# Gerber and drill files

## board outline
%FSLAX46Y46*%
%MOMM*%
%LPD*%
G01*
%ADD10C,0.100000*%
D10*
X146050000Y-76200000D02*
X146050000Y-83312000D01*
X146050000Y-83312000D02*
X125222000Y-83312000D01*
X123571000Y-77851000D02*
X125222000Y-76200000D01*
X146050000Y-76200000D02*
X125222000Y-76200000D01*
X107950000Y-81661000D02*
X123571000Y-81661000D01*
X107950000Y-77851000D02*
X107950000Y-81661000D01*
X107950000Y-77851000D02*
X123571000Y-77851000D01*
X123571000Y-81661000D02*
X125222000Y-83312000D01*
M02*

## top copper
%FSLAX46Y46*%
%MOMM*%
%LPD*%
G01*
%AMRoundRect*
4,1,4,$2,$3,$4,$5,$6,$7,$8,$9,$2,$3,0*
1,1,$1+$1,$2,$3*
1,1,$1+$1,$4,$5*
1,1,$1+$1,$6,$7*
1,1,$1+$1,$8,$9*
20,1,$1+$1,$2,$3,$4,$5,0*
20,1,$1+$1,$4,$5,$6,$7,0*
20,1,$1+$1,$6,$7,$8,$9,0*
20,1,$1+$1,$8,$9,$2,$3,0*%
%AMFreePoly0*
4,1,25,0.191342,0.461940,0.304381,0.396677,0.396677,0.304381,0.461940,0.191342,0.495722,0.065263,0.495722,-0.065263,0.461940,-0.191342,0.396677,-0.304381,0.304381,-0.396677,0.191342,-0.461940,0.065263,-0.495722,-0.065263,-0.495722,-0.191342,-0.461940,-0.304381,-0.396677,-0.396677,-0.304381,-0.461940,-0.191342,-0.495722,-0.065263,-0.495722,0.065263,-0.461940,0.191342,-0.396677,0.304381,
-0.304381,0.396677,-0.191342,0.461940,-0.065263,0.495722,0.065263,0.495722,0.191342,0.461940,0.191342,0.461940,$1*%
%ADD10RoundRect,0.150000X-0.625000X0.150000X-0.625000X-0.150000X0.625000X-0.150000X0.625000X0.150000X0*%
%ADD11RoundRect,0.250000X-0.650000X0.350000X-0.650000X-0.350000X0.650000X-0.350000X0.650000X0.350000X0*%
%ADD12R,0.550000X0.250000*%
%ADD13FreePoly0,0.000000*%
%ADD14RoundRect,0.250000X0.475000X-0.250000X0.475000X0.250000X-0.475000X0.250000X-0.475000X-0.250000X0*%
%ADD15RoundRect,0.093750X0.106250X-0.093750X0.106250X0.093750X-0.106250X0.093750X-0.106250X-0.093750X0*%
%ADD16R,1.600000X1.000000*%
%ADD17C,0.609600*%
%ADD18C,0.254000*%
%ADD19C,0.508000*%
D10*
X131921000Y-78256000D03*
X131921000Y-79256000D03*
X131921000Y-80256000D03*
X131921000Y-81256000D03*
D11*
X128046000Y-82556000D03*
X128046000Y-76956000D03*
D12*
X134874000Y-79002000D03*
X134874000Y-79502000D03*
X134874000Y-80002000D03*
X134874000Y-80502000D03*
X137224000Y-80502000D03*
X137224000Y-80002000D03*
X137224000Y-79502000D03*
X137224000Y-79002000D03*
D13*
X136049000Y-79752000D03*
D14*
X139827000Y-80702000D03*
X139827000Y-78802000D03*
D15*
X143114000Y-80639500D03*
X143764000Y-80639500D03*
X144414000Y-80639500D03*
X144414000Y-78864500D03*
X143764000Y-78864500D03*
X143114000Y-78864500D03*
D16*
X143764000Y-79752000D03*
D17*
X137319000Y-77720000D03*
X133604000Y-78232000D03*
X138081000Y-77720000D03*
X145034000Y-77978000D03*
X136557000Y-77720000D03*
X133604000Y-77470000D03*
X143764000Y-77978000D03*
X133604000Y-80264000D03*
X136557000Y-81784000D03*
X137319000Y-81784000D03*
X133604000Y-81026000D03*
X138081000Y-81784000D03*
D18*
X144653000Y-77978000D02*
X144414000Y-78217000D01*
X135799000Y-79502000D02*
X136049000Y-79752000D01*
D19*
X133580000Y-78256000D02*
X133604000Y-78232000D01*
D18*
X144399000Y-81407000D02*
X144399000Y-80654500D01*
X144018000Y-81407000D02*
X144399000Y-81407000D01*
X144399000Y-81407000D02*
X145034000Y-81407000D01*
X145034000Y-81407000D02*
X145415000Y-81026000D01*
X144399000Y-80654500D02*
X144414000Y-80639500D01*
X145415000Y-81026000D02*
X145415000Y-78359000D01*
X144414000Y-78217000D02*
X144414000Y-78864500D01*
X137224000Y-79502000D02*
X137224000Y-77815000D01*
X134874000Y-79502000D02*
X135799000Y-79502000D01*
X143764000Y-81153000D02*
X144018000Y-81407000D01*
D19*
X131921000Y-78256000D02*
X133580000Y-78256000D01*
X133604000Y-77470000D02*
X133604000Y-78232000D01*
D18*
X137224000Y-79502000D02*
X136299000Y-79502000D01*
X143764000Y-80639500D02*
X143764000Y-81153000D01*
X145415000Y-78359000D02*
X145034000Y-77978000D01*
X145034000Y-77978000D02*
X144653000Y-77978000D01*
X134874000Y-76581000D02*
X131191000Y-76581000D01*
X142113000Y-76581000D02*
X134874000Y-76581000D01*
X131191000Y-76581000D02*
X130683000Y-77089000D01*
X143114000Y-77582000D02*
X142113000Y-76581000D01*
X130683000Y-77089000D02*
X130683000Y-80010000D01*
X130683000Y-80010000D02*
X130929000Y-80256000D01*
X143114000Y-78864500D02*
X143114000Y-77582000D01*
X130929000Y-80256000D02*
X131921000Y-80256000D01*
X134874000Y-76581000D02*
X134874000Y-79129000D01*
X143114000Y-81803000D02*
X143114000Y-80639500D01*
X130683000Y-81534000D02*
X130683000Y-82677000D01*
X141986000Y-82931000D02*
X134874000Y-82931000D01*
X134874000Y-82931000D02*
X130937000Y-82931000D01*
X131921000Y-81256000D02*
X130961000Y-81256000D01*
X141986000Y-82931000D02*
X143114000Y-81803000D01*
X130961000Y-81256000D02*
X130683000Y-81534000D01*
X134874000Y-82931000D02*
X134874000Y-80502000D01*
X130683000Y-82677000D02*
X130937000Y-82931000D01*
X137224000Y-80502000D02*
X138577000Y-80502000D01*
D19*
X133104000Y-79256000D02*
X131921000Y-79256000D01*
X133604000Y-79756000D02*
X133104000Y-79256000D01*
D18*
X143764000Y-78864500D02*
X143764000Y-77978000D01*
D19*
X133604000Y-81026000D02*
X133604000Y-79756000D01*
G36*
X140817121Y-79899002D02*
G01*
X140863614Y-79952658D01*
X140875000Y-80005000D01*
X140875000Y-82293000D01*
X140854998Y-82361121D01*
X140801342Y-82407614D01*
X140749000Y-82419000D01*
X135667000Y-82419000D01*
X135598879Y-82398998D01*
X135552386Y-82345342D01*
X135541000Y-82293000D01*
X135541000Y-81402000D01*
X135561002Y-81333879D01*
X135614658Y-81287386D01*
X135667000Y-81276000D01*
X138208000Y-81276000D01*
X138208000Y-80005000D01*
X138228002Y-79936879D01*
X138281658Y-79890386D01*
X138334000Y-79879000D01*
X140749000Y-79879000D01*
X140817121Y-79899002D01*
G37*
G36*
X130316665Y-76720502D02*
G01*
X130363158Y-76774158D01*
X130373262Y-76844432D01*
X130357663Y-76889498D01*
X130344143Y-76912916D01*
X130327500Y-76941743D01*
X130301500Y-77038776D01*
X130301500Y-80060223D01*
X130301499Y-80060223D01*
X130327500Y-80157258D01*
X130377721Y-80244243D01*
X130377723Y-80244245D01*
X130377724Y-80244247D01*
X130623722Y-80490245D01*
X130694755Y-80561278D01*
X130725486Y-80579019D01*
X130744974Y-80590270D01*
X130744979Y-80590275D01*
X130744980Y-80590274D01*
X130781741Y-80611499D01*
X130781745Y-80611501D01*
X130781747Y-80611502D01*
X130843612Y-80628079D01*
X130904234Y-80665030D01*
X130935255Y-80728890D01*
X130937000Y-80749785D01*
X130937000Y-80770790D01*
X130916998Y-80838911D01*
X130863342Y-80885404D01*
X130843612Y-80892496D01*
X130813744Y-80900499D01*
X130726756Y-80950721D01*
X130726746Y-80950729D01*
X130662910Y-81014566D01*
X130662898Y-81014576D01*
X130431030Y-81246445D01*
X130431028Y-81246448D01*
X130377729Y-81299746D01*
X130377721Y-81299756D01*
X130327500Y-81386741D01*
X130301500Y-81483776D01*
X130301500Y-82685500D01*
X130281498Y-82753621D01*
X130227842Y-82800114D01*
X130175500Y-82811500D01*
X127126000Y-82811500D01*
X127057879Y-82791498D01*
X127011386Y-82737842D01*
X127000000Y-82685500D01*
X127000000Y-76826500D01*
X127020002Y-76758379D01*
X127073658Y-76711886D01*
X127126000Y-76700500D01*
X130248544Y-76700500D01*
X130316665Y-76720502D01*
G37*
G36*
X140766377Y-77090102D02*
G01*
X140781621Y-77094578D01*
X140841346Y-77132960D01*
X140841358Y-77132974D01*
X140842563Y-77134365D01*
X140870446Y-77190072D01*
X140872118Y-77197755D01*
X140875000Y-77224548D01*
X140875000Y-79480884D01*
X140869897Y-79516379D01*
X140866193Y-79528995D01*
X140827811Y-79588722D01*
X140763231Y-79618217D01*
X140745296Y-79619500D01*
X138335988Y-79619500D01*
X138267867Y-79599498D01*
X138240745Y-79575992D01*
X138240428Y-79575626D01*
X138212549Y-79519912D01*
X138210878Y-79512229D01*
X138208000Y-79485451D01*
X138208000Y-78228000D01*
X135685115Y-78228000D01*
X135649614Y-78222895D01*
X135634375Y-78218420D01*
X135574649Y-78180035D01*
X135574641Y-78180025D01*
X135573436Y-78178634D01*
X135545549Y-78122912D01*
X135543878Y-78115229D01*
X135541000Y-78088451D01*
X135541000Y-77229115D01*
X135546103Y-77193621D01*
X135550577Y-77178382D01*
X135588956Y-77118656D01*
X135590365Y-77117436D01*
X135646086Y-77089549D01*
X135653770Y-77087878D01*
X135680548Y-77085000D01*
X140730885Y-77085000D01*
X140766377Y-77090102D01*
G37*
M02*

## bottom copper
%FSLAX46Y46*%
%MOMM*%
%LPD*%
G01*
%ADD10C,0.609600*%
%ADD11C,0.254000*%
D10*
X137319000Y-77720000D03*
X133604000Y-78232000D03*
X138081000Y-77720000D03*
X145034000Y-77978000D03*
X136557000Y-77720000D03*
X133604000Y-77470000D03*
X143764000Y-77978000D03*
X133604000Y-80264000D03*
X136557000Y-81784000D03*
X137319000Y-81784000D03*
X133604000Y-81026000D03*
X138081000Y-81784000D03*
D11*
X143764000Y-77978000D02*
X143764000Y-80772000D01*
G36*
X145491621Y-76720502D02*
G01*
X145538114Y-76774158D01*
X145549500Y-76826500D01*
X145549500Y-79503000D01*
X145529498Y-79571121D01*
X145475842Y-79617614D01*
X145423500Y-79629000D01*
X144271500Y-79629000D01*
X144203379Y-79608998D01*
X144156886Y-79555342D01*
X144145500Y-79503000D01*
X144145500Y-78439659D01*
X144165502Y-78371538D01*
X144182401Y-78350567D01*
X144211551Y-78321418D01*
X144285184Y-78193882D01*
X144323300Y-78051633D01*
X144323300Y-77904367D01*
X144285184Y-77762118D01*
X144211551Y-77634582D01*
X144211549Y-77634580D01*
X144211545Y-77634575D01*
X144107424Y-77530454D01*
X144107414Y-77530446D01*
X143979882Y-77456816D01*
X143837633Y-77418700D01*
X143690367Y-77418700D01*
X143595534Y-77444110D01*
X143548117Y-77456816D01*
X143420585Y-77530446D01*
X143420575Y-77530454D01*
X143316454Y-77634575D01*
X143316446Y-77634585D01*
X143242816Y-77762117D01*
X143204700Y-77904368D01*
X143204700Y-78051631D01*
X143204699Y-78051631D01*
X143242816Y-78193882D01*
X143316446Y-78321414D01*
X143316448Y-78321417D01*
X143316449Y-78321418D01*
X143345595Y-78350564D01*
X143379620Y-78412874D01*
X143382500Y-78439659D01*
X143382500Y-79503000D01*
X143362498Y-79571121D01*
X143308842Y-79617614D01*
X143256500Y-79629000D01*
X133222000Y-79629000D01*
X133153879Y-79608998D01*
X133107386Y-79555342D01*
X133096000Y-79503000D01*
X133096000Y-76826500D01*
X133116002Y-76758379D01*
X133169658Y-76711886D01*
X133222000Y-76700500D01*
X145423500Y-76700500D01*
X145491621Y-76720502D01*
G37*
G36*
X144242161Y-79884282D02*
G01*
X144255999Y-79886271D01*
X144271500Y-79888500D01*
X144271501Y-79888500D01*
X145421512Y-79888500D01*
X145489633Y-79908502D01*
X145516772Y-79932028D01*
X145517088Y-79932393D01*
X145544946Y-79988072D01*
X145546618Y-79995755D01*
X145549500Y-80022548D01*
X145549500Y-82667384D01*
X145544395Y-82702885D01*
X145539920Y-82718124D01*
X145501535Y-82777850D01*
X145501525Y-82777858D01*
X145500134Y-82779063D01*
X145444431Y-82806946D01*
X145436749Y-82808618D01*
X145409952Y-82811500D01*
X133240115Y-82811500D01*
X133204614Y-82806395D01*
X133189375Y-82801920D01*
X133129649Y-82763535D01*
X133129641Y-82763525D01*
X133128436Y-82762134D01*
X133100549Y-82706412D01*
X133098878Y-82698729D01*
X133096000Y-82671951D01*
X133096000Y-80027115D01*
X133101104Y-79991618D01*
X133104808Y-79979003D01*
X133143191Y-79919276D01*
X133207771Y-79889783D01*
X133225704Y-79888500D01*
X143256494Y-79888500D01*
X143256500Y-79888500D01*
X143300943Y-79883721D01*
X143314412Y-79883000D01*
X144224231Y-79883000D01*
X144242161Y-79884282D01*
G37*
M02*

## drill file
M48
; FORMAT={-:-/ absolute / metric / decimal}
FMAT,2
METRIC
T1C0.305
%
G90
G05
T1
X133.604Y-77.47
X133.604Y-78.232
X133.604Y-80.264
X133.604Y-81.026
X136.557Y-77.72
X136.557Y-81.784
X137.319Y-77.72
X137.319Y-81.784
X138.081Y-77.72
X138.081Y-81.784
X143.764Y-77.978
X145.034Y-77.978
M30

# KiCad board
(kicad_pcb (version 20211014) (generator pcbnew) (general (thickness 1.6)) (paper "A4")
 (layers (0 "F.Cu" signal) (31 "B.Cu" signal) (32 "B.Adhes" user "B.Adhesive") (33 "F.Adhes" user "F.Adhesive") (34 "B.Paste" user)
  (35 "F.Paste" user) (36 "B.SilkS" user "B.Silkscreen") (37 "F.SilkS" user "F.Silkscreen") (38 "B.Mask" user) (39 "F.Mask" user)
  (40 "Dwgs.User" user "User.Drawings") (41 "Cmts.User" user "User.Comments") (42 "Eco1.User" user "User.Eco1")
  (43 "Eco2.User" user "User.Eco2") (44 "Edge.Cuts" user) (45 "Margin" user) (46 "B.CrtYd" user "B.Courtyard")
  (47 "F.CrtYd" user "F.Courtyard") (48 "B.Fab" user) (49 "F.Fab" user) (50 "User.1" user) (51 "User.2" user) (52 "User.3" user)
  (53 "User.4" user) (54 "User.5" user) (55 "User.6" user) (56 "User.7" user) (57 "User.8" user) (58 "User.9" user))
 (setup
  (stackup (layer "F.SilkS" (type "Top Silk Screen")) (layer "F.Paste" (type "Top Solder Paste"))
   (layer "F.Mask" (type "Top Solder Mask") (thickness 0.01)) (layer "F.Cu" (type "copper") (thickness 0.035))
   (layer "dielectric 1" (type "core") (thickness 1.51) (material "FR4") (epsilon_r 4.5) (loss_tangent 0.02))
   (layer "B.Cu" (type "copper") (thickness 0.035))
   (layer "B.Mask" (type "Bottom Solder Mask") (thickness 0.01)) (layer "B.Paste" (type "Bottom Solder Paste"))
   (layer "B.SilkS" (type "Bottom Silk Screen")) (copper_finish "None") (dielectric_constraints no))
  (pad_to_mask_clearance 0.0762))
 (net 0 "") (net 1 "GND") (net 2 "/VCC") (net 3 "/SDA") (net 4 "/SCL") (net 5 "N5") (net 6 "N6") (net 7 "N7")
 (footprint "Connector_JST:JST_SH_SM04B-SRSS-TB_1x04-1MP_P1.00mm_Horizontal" (layer "F.Cu") (at 129.921 79.756 -90)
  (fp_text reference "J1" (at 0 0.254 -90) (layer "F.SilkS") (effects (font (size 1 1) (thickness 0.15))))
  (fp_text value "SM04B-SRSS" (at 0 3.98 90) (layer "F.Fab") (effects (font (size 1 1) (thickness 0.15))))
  (pad "1" smd roundrect (at -1.5 -2 270) (size 0.6 1.55) (layers "F.Cu" "F.Paste" "F.Mask") (roundrect_rratio 0.25) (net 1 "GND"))
  (pad "2" smd roundrect (at -0.5 -2 270) (size 0.6 1.55) (layers "F.Cu" "F.Paste" "F.Mask") (roundrect_rratio 0.25) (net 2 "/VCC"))
  (pad "3" smd roundrect (at 0.5 -2 270) (size 0.6 1.55) (layers "F.Cu" "F.Paste" "F.Mask") (roundrect_rratio 0.25) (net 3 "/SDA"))
  (pad "4" smd roundrect (at 1.5 -2 270) (size 0.6 1.55) (layers "F.Cu" "F.Paste" "F.Mask") (roundrect_rratio 0.25) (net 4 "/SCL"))
  (pad "MP" smd roundrect (at 2.8 1.875 270) (size 1.2 1.8) (layers "F.Cu" "F.Paste" "F.Mask") (roundrect_rratio 0.208333) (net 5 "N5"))
  (pad "MP" smd roundrect (at -2.8 1.875 270) (size 1.2 1.8) (layers "F.Cu" "F.Paste" "F.Mask") (roundrect_rratio 0.208333) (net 5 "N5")))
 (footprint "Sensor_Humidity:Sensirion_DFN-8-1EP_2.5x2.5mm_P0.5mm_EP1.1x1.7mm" (layer "F.Cu") (at 136.049 79.752)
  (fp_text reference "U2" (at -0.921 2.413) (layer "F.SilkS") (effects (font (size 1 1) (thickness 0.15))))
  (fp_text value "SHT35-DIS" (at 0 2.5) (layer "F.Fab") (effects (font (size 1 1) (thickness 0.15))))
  (pad "" smd custom (at 0 0) (size 0.9 0.9) (layers "F.Paste") (zone_connect 0) (options (clearance outline) (anchor rect)) (primitives))
  (pad "1" smd rect (at -1.175 -0.75) (size 0.55 0.25) (layers "F.Cu" "F.Paste" "F.Mask") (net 3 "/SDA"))
  (pad "2" smd rect (at -1.175 -0.25) (size 0.55 0.25) (layers "F.Cu" "F.Paste" "F.Mask") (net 1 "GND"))
  (pad "3" smd rect (at -1.175 0.25) (size 0.55 0.25) (layers "F.Cu" "F.Paste" "F.Mask") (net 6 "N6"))
  (pad "4" smd rect (at -1.175 0.75 180) (size 0.55 0.25) (layers "F.Cu" "F.Paste" "F.Mask") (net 4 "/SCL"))
  (pad "5" smd rect (at 1.175 0.75) (size 0.55 0.25) (layers "F.Cu" "F.Paste" "F.Mask") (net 2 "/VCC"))
  (pad "6" smd rect (at 1.175 0.25) (size 0.55 0.25) (layers "F.Cu" "F.Paste" "F.Mask") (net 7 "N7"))
  (pad "7" smd rect (at 1.175 -0.25) (size 0.55 0.25) (layers "F.Cu" "F.Paste" "F.Mask") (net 1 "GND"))
  (pad "8" smd rect (at 1.175 -0.75) (size 0.55 0.25) (layers "F.Cu" "F.Paste" "F.Mask") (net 1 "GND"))
  (pad "9" smd custom (at 0 0) (size 1 1) (layers "F.Cu" "F.Mask") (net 1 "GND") (zone_connect 0)
   (options (clearance outline) (anchor circle)) (primitives)))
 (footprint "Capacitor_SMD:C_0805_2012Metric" (layer "F.Cu") (at 139.827 79.752 90)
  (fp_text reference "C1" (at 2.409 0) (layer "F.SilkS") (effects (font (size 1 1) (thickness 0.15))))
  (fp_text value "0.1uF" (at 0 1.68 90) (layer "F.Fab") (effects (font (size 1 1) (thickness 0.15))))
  (pad "1" smd roundrect (at -0.95 0 90) (size 1 1.45) (layers "F.Cu" "F.Paste" "F.Mask") (roundrect_rratio 0.25) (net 2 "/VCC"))
  (pad "2" smd roundrect (at 0.95 0 90) (size 1 1.45) (layers "F.Cu" "F.Paste" "F.Mask") (roundrect_rratio 0.25) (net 1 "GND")))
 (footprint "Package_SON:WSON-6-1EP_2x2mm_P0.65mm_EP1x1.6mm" (layer "F.Cu") (at 143.764 79.752 90)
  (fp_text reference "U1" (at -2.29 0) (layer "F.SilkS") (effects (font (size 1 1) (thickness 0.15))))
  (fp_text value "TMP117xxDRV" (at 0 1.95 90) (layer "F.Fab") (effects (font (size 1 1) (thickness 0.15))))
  (pad "1" smd roundrect (at -0.8875 -0.65 90) (size 0.375 0.4) (layers "F.Cu" "F.Paste" "F.Mask") (roundrect_rratio 0.25) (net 4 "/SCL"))
  (pad "2" smd roundrect (at -0.8875 0 90) (size 0.375 0.4) (layers "F.Cu" "F.Paste" "F.Mask") (roundrect_rratio 0.25) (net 1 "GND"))
  (pad "3" smd roundrect (at -0.8875 0.65 90) (size 0.375 0.4) (layers "F.Cu" "F.Paste" "F.Mask") (roundrect_rratio 0.25) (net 1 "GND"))
  (pad "4" smd roundrect (at 0.8875 0.65 90) (size 0.375 0.4) (layers "F.Cu" "F.Paste" "F.Mask") (roundrect_rratio 0.25) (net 1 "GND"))
  (pad "5" smd roundrect (at 0.8875 0 90) (size 0.375 0.4) (layers "F.Cu" "F.Paste" "F.Mask") (roundrect_rratio 0.25) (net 2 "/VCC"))
  (pad "6" smd roundrect (at 0.8875 -0.65 90) (size 0.375 0.4) (layers "F.Cu" "F.Paste" "F.Mask") (roundrect_rratio 0.25) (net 3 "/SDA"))
  (pad "7" smd rect (at 0 0 90) (size 1 1.6) (layers "F.Cu" "F.Mask")))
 (gr_line (start 146.05 76.2) (end 146.05 83.312) (layer "Edge.Cuts") (width 0.1))
 (gr_line (start 146.05 83.312) (end 125.222 83.312) (layer "Edge.Cuts") (width 0.1))
 (gr_line (start 123.571 77.851) (end 125.222 76.2) (layer "Edge.Cuts") (width 0.1))
 (gr_line (start 146.05 76.2) (end 125.222 76.2) (layer "Edge.Cuts") (width 0.1))
 (gr_line (start 107.95 81.661) (end 123.571 81.661) (layer "Edge.Cuts") (width 0.1))
 (gr_line (start 107.95 77.851) (end 107.95 81.661) (layer "Edge.Cuts") (width 0.1))
 (gr_line (start 107.95 77.851) (end 123.571 77.851) (layer "Edge.Cuts") (width 0.1))
 (gr_line (start 123.571 81.661) (end 125.222 83.312) (layer "Edge.Cuts") (width 0.1))
 (segment (start 144.653 77.978) (end 144.414 78.217) (width 0.254) (layer "F.Cu") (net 1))
 (segment (start 135.799 79.502) (end 136.049 79.752) (width 0.254) (layer "F.Cu") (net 1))
 (segment (start 133.58 78.256) (end 133.604 78.232) (width 0.508) (layer "F.Cu") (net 1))
 (segment (start 144.399 81.407) (end 144.399 80.6545) (width 0.254) (layer "F.Cu") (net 1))
 (segment (start 144.018 81.407) (end 144.399 81.407) (width 0.254) (layer "F.Cu") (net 1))
 (segment (start 144.399 81.407) (end 145.034 81.407) (width 0.254) (layer "F.Cu") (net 1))
 (segment (start 145.034 81.407) (end 145.415 81.026) (width 0.254) (layer "F.Cu") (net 1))
 (segment (start 144.399 80.6545) (end 144.414 80.6395) (width 0.254) (layer "F.Cu") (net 1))
 (segment (start 145.415 81.026) (end 145.415 78.359) (width 0.254) (layer "F.Cu") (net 1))
 (segment (start 144.414 78.217) (end 144.414 78.8645) (width 0.254) (layer "F.Cu") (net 1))
 (segment (start 137.224 79.502) (end 137.224 77.815) (width 0.254) (layer "F.Cu") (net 1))
 (segment (start 134.874 79.502) (end 135.799 79.502) (width 0.254) (layer "F.Cu") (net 1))
 (segment (start 143.764 81.153) (end 144.018 81.407) (width 0.254) (layer "F.Cu") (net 1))
 (segment (start 131.921 78.256) (end 133.58 78.256) (width 0.508) (layer "F.Cu") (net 1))
 (segment (start 133.604 77.47) (end 133.604 78.232) (width 0.508) (layer "F.Cu") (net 1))
 (segment (start 137.224 79.502) (end 136.299 79.502) (width 0.254) (layer "F.Cu") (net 1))
 (segment (start 143.764 80.6395) (end 143.764 81.153) (width 0.254) (layer "F.Cu") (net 1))
 (segment (start 145.415 78.359) (end 145.034 77.978) (width 0.254) (layer "F.Cu") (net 1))
 (segment (start 145.034 77.978) (end 144.653 77.978) (width 0.254) (layer "F.Cu") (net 1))
 (via (at 137.319 77.72) (size 0.6096) (drill 0.3048) (layers "F.Cu" "B.Cu") (free) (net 1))
 (via (at 133.604 78.232) (size 0.6096) (drill 0.3048) (layers "F.Cu" "B.Cu") (free) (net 1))
 (via (at 138.081 77.72) (size 0.6096) (drill 0.3048) (layers "F.Cu" "B.Cu") (free) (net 1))
 (via (at 145.034 77.978) (size 0.6096) (drill 0.3048) (layers "F.Cu" "B.Cu") (free) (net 1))
 (via (at 136.557 77.72) (size 0.6096) (drill 0.3048) (layers "F.Cu" "B.Cu") (free) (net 1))
 (via (at 133.604 77.47) (size 0.6096) (drill 0.3048) (layers "F.Cu" "B.Cu") (free) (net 1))
 (segment (start 134.874 76.581) (end 131.191 76.581) (width 0.254) (layer "F.Cu") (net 3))
 (segment (start 142.113 76.581) (end 134.874 76.581) (width 0.254) (layer "F.Cu") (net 3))
 (segment (start 131.191 76.581) (end 130.683 77.089) (width 0.254) (layer "F.Cu") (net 3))
 (segment (start 143.114 77.582) (end 142.113 76.581) (width 0.254) (layer "F.Cu") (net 3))
 (segment (start 130.683 77.089) (end 130.683 80.01) (width 0.254) (layer "F.Cu") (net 3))
 (segment (start 130.683 80.01) (end 130.929 80.256) (width 0.254) (layer "F.Cu") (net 3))
 (segment (start 143.114 78.8645) (end 143.114 77.582) (width 0.254) (layer "F.Cu") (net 3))
 (segment (start 130.929 80.256) (end 131.921 80.256) (width 0.254) (layer "F.Cu") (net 3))
 (segment (start 134.874 76.581) (end 134.874 79.129) (width 0.254) (layer "F.Cu") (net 3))
 (segment (start 143.114 81.803) (end 143.114 80.6395) (width 0.254) (layer "F.Cu") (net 4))
 (segment (start 130.683 81.534) (end 130.683 82.677) (width 0.254) (layer "F.Cu") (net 4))
 (segment (start 141.986 82.931) (end 134.874 82.931) (width 0.254) (layer "F.Cu") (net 4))
 (segment (start 134.874 82.931) (end 130.937 82.931) (width 0.254) (layer "F.Cu") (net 4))
 (segment (start 131.921 81.256) (end 130.961 81.256) (width 0.254) (layer "F.Cu") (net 4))
 (segment (start 141.986 82.931) (end 143.114 81.803) (width 0.254) (layer "F.Cu") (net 4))
 (segment (start 130.961 81.256) (end 130.683 81.534) (width 0.254) (layer "F.Cu") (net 4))
 (segment (start 134.874 82.931) (end 134.874 80.502) (width 0.254) (layer "F.Cu") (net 4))
 (segment (start 130.683 82.677) (end 130.937 82.931) (width 0.254) (layer "F.Cu") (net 4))
 (segment (start 137.224 80.502) (end 138.577 80.502) (width 0.254) (layer "F.Cu") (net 2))
 (segment (start 133.104 79.256) (end 131.921 79.256) (width 0.508) (layer "F.Cu") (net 2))
 (segment (start 133.604 79.756) (end 133.104 79.256) (width 0.508) (layer "F.Cu") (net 2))
 (segment (start 143.764 78.8645) (end 143.764 77.978) (width 0.254) (layer "F.Cu") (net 2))
 (segment (start 133.604 81.026) (end 133.604 79.756) (width 0.508) (layer "F.Cu") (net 2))
 (via (at 143.764 77.978) (size 0.6096) (drill 0.3048) (layers "F.Cu" "B.Cu") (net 2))
 (via (at 133.604 80.264) (size 0.6096) (drill 0.3048) (layers "F.Cu" "B.Cu") (free) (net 2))
 (via (at 136.557 81.784) (size 0.6096) (drill 0.3048) (layers "F.Cu" "B.Cu") (free) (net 2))
 (via (at 137.319 81.784) (size 0.6096) (drill 0.3048) (layers "F.Cu" "B.Cu") (free) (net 2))
 (via (at 133.604 81.026) (size 0.6096) (drill 0.3048) (layers "F.Cu" "B.Cu") (free) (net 2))
 (via (at 138.081 81.784) (size 0.6096) (drill 0.3048) (layers "F.Cu" "B.Cu") (free) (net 2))
 (segment (start 143.764 77.978) (end 143.764 80.772) (width 0.254) (layer "B.Cu") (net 2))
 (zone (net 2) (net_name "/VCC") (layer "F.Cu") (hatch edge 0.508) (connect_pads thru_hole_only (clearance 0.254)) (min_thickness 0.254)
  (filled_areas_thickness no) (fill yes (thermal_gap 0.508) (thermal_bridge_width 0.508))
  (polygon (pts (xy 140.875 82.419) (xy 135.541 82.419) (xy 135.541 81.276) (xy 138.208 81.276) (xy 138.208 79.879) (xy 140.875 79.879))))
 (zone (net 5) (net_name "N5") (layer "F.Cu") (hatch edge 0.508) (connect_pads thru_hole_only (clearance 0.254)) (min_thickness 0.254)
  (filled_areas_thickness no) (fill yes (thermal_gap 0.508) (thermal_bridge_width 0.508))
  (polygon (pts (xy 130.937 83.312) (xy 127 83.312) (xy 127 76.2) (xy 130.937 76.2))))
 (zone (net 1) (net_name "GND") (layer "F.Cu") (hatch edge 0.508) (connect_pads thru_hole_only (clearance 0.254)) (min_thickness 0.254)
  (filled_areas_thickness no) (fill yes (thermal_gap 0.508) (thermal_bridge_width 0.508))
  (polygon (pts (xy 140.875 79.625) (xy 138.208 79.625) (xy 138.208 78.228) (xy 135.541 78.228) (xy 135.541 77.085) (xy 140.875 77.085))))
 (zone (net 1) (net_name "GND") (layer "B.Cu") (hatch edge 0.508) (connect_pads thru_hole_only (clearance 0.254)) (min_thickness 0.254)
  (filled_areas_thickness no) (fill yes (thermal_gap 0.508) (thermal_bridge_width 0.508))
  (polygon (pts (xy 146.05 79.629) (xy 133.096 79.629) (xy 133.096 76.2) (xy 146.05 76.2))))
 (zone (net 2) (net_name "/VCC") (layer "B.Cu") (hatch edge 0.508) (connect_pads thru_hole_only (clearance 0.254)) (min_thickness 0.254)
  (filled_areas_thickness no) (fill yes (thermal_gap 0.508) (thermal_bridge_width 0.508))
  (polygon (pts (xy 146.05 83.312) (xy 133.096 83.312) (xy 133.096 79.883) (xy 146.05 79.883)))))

